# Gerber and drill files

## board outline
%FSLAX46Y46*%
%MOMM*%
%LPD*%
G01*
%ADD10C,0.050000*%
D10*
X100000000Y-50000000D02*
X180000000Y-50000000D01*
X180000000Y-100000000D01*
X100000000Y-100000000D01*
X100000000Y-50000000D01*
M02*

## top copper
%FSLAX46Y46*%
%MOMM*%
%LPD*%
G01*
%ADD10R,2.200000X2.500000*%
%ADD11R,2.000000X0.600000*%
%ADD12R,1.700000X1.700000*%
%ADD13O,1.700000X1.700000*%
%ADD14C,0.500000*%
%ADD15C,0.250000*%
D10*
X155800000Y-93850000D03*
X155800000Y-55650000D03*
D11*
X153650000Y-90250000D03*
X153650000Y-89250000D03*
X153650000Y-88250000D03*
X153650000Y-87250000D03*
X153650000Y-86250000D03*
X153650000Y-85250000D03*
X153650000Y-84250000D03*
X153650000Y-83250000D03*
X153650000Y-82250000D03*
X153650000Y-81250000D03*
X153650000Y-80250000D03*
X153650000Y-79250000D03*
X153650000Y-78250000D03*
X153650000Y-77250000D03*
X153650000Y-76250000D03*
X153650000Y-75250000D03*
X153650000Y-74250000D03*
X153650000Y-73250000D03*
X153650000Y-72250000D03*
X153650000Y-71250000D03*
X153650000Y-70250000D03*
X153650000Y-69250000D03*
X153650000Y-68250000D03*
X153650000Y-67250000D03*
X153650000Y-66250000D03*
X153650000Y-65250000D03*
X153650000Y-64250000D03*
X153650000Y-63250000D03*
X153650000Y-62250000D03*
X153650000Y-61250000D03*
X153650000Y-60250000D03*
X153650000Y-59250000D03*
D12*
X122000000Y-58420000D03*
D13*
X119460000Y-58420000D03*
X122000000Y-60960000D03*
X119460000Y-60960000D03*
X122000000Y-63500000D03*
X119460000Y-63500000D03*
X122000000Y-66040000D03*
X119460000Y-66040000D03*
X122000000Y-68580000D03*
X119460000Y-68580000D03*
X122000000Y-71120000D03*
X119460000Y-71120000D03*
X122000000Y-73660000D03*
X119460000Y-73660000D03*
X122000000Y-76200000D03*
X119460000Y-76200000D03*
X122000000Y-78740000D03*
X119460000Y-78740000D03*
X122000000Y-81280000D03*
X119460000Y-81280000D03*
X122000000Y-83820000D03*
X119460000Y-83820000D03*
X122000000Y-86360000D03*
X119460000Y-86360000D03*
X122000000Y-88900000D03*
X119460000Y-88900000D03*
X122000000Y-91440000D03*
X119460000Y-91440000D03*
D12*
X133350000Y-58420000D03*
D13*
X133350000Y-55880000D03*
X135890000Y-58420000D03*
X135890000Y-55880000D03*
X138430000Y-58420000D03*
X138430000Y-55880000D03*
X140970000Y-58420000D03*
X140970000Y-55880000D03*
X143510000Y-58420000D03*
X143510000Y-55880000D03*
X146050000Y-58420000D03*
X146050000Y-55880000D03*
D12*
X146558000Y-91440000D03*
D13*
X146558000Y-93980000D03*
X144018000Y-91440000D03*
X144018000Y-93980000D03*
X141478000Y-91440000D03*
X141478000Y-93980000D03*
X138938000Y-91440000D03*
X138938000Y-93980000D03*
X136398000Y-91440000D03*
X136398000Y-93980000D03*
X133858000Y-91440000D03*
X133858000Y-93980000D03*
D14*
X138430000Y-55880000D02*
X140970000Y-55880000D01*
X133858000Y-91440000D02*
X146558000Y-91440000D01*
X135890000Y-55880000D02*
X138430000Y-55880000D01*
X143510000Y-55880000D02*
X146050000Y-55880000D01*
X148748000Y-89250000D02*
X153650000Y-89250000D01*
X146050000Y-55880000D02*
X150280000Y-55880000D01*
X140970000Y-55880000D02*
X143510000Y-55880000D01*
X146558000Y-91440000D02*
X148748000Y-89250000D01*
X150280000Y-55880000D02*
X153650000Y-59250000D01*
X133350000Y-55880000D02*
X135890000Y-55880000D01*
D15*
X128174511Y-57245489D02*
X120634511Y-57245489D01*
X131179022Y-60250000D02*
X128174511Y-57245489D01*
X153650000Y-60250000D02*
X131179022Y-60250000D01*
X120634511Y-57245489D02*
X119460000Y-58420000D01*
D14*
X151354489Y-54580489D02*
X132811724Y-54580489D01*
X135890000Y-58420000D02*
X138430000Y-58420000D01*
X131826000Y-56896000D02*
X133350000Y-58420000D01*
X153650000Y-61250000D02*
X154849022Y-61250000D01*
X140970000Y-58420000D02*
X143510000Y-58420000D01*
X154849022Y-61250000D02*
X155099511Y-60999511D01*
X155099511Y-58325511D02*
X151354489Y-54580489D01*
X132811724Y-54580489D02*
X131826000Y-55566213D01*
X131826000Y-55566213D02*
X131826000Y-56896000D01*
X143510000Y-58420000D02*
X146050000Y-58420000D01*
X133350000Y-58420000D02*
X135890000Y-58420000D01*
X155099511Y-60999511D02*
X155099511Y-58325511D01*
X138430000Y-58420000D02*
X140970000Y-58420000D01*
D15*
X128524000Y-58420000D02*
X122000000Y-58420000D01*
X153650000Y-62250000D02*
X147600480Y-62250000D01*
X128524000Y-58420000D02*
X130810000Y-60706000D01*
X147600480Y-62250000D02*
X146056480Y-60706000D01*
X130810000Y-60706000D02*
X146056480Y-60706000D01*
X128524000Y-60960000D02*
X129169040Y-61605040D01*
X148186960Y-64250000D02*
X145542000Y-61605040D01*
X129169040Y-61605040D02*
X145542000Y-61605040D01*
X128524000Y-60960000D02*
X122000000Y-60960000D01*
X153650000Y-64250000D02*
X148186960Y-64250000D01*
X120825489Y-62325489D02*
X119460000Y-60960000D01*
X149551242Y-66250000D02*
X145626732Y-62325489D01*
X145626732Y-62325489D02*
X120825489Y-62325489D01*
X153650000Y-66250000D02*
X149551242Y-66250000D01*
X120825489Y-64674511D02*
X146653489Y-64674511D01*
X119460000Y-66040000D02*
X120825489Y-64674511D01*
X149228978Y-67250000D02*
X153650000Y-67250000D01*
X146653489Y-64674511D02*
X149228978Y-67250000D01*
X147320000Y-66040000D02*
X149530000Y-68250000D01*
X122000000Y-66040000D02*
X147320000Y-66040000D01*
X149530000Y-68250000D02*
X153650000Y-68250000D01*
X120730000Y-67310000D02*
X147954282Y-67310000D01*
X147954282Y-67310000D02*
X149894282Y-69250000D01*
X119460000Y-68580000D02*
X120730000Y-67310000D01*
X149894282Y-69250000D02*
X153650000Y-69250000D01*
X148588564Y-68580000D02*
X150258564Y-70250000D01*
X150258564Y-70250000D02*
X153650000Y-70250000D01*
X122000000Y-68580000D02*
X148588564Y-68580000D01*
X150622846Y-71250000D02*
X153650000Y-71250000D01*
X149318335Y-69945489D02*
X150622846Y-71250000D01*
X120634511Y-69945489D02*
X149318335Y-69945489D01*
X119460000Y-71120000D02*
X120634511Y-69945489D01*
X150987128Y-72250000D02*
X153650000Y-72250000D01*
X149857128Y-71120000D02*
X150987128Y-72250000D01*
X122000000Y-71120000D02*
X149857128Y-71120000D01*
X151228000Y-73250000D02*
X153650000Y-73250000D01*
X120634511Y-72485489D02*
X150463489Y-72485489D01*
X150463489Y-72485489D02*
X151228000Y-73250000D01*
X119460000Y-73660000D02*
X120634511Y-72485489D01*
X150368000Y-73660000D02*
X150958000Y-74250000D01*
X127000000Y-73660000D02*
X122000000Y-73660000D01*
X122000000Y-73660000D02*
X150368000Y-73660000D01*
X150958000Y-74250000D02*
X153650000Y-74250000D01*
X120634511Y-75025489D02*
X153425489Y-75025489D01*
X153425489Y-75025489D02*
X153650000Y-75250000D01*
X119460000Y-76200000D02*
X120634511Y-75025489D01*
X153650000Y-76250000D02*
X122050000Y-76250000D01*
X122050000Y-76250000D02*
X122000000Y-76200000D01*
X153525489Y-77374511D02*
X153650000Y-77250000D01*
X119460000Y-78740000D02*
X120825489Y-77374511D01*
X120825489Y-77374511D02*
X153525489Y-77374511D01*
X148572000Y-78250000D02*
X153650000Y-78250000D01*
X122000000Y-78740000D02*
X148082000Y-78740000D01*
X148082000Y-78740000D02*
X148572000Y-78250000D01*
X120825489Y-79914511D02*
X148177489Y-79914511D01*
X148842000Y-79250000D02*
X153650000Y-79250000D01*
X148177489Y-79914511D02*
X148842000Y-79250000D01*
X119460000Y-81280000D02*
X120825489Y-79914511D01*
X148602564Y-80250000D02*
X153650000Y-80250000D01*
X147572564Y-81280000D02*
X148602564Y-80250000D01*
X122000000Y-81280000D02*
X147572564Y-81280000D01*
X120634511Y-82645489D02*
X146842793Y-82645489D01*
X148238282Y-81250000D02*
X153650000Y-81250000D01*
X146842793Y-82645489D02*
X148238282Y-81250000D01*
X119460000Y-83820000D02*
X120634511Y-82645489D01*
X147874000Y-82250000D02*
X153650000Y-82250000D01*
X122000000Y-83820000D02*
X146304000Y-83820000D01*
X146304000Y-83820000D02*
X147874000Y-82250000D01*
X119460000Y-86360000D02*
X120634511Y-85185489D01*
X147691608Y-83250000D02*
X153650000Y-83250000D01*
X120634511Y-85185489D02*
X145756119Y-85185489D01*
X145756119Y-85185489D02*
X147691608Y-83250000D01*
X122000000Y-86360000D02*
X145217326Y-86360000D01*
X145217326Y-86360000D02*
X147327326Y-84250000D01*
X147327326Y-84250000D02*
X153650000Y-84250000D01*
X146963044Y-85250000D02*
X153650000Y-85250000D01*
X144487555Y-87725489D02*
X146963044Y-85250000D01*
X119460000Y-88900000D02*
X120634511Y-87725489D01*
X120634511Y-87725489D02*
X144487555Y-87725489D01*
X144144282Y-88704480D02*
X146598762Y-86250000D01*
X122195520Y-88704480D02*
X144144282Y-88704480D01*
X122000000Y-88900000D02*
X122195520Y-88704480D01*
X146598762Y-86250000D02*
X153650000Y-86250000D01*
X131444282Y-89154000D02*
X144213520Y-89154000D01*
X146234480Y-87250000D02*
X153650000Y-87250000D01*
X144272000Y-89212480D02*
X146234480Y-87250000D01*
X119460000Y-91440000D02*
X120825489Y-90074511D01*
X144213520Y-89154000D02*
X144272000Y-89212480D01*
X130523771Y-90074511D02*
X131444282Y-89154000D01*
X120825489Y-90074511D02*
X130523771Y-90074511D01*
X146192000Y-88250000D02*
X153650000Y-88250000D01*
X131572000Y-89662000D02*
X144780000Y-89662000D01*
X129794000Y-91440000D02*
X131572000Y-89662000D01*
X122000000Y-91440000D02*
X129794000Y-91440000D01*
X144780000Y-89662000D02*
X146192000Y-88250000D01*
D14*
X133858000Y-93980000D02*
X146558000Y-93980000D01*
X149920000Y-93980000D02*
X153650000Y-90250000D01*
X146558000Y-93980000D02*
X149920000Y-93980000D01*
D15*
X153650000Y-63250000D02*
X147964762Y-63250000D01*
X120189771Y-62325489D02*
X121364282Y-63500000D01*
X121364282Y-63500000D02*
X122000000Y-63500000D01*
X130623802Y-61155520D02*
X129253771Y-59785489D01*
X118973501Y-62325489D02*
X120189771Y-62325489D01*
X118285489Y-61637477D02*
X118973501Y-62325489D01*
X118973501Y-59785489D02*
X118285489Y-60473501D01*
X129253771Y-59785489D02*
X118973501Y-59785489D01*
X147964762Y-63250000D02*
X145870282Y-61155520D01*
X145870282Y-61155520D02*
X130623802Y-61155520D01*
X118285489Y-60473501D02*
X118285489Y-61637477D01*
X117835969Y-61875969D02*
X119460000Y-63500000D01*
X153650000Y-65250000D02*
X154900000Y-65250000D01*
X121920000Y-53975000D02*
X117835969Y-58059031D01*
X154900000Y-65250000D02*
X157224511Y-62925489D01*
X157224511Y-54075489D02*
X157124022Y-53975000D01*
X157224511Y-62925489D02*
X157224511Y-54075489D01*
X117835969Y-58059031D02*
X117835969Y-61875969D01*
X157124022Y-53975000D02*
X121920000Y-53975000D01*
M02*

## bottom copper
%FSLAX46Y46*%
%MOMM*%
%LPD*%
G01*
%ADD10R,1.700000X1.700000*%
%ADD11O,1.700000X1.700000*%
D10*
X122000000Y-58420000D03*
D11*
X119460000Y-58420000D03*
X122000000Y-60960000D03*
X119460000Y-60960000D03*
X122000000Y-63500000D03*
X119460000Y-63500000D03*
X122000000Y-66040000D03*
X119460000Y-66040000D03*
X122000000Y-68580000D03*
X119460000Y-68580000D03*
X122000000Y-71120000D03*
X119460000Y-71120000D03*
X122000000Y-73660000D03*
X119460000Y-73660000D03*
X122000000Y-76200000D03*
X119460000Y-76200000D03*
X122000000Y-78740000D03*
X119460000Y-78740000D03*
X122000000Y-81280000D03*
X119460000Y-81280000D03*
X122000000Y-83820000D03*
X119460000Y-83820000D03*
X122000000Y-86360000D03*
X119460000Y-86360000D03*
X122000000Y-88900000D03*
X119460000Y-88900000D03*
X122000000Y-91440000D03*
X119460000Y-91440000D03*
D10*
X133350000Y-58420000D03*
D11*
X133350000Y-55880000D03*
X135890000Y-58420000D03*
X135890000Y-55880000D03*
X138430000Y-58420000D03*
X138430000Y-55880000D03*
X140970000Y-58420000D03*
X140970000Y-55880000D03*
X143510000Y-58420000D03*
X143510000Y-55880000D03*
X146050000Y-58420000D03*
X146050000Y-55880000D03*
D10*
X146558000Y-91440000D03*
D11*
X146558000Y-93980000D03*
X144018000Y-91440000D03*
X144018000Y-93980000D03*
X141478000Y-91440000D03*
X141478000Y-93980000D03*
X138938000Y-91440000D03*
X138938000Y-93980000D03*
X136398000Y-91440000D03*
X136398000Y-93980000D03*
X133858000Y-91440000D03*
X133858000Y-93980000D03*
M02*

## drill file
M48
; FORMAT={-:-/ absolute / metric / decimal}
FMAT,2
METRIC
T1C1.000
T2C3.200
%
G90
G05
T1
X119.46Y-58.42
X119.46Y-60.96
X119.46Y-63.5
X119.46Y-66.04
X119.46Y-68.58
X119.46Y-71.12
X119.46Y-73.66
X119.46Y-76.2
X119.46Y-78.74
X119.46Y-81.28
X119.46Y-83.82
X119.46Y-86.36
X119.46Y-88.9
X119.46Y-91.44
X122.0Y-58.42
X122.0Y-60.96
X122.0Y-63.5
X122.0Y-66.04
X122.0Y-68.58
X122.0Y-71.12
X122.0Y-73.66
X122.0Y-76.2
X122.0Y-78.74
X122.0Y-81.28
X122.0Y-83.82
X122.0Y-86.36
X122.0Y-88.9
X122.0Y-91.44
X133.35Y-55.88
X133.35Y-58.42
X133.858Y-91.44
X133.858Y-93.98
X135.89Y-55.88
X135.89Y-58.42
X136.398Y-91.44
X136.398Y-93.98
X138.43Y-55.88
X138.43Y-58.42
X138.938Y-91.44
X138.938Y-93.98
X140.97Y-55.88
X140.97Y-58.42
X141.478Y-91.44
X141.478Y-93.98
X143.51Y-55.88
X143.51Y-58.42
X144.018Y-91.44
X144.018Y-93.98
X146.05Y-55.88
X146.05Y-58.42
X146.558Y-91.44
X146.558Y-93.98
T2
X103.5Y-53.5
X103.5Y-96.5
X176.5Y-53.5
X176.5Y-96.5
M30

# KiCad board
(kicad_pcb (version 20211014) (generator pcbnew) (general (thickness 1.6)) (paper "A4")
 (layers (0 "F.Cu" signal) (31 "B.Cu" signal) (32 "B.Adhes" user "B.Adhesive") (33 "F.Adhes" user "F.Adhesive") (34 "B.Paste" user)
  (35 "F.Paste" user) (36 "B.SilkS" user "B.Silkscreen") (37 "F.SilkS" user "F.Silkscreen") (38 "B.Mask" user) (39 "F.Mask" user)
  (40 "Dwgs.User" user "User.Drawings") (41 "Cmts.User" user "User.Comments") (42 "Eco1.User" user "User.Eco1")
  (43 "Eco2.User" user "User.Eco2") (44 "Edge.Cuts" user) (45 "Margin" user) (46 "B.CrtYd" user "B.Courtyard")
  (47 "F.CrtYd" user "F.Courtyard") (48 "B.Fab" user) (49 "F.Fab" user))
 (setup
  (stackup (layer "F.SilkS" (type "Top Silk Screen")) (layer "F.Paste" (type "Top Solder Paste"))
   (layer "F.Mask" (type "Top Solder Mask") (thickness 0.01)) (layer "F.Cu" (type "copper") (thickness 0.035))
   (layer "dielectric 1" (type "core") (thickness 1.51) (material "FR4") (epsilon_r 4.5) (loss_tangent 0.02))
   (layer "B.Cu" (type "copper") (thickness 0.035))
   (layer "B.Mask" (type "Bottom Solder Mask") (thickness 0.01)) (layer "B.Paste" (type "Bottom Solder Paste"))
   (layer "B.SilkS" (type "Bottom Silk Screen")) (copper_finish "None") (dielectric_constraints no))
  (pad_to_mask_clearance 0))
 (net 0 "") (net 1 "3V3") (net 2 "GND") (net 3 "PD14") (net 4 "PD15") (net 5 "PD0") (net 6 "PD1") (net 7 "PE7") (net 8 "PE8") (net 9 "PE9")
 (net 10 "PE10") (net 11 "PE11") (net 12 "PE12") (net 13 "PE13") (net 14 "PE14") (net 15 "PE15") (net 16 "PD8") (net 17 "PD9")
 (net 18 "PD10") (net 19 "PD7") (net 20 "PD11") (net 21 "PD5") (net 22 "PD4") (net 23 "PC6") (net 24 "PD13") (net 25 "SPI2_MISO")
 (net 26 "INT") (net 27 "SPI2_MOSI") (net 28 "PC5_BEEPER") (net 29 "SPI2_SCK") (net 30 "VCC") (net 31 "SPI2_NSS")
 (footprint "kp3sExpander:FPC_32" (layer "F.Cu") (at 153.65 74.75 90)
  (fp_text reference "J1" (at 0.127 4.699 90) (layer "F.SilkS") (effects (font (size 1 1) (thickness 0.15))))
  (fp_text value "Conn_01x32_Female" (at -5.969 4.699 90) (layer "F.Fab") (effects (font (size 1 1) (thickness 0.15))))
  (pad "0" smd rect locked (at -19.1 2.15 90) (size 2.5 2.2) (layers "F.Cu" "F.Paste" "F.Mask"))
  (pad "0" smd rect locked (at 19.1 2.15 90) (size 2.5 2.2) (layers "F.Cu" "F.Paste" "F.Mask"))
  (pad "1" smd rect locked (at -15.5 0 90) (size 0.6 2) (layers "F.Cu" "F.Paste" "F.Mask") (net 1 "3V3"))
  (pad "2" smd rect locked (at -14.5 0 90) (size 0.6 2) (layers "F.Cu" "F.Paste" "F.Mask") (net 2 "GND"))
  (pad "3" smd rect locked (at -13.5 0 90) (size 0.6 2) (layers "F.Cu" "F.Paste" "F.Mask") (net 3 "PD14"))
  (pad "4" smd rect locked (at -12.5 0 90) (size 0.6 2) (layers "F.Cu" "F.Paste" "F.Mask") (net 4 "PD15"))
  (pad "5" smd rect locked (at -11.5 0 90) (size 0.6 2) (layers "F.Cu" "F.Paste" "F.Mask") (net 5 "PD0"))
  (pad "6" smd rect locked (at -10.5 0 90) (size 0.6 2) (layers "F.Cu" "F.Paste" "F.Mask") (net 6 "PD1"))
  (pad "7" smd rect locked (at -9.5 0 90) (size 0.6 2) (layers "F.Cu" "F.Paste" "F.Mask") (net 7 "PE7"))
  (pad "8" smd rect locked (at -8.5 0 90) (size 0.6 2) (layers "F.Cu" "F.Paste" "F.Mask") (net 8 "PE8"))
  (pad "9" smd rect locked (at -7.5 0 90) (size 0.6 2) (layers "F.Cu" "F.Paste" "F.Mask") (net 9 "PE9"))
  (pad "10" smd rect locked (at -6.5 0 90) (size 0.6 2) (layers "F.Cu" "F.Paste" "F.Mask") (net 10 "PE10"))
  (pad "11" smd rect locked (at -5.5 0 90) (size 0.6 2) (layers "F.Cu" "F.Paste" "F.Mask") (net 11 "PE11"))
  (pad "12" smd rect locked (at -4.5 0 90) (size 0.6 2) (layers "F.Cu" "F.Paste" "F.Mask") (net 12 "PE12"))
  (pad "13" smd rect locked (at -3.5 0 90) (size 0.6 2) (layers "F.Cu" "F.Paste" "F.Mask") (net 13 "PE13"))
  (pad "14" smd rect locked (at -2.5 0 90) (size 0.6 2) (layers "F.Cu" "F.Paste" "F.Mask") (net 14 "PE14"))
  (pad "15" smd rect locked (at -1.5 0 90) (size 0.6 2) (layers "F.Cu" "F.Paste" "F.Mask") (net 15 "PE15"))
  (pad "16" smd rect locked (at -0.5 0 90) (size 0.6 2) (layers "F.Cu" "F.Paste" "F.Mask") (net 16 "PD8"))
  (pad "17" smd rect locked (at 0.5 0 90) (size 0.6 2) (layers "F.Cu" "F.Paste" "F.Mask") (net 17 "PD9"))
  (pad "18" smd rect locked (at 1.5 0 90) (size 0.6 2) (layers "F.Cu" "F.Paste" "F.Mask") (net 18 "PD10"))
  (pad "19" smd rect locked (at 2.5 0 90) (size 0.6 2) (layers "F.Cu" "F.Paste" "F.Mask") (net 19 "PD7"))
  (pad "20" smd rect locked (at 3.5 0 90) (size 0.6 2) (layers "F.Cu" "F.Paste" "F.Mask") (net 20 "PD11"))
  (pad "21" smd rect locked (at 4.5 0 90) (size 0.6 2) (layers "F.Cu" "F.Paste" "F.Mask") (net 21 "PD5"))
  (pad "22" smd rect locked (at 5.5 0 90) (size 0.6 2) (layers "F.Cu" "F.Paste" "F.Mask") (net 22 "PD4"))
  (pad "23" smd rect locked (at 6.5 0 90) (size 0.6 2) (layers "F.Cu" "F.Paste" "F.Mask") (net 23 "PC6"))
  (pad "24" smd rect locked (at 7.5 0 90) (size 0.6 2) (layers "F.Cu" "F.Paste" "F.Mask") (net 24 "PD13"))
  (pad "25" smd rect locked (at 8.5 0 90) (size 0.6 2) (layers "F.Cu" "F.Paste" "F.Mask") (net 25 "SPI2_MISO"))
  (pad "26" smd rect locked (at 9.5 0 90) (size 0.6 2) (layers "F.Cu" "F.Paste" "F.Mask") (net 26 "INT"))
  (pad "27" smd rect locked (at 10.5 0 90) (size 0.6 2) (layers "F.Cu" "F.Paste" "F.Mask") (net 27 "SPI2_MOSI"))
  (pad "28" smd rect locked (at 11.5 0 90) (size 0.6 2) (layers "F.Cu" "F.Paste" "F.Mask") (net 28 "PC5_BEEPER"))
  (pad "29" smd rect locked (at 12.5 0 90) (size 0.6 2) (layers "F.Cu" "F.Paste" "F.Mask") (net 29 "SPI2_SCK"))
  (pad "30" smd rect locked (at 13.5 0 90) (size 0.6 2) (layers "F.Cu" "F.Paste" "F.Mask") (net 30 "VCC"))
  (pad "31" smd rect locked (at 14.5 0 90) (size 0.6 2) (layers "F.Cu" "F.Paste" "F.Mask") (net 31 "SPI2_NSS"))
  (pad "32" smd rect locked (at 15.5 0 90) (size 0.6 2) (layers "F.Cu" "F.Paste" "F.Mask") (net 2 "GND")))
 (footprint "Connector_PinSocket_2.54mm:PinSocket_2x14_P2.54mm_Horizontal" (layer "F.Cu") (at 122 58.42)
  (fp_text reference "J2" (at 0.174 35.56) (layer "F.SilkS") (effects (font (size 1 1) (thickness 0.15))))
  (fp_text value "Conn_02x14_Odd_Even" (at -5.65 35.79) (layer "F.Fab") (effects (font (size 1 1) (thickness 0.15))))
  (pad "1" thru_hole rect (at 0 0) (size 1.7 1.7) (drill 1) (layers *.Cu *.Mask) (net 29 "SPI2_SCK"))
  (pad "2" thru_hole oval (at -2.54 0) (size 1.7 1.7) (drill 1) (layers *.Cu *.Mask) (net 31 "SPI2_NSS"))
  (pad "3" thru_hole oval (at 0 2.54) (size 1.7 1.7) (drill 1) (layers *.Cu *.Mask) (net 27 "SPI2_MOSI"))
  (pad "4" thru_hole oval (at -2.54 2.54) (size 1.7 1.7) (drill 1) (layers *.Cu *.Mask) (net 25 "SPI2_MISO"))
  (pad "5" thru_hole oval (at 0 5.08) (size 1.7 1.7) (drill 1) (layers *.Cu *.Mask) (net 28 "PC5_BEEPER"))
  (pad "6" thru_hole oval (at -2.54 5.08) (size 1.7 1.7) (drill 1) (layers *.Cu *.Mask) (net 26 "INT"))
  (pad "7" thru_hole oval (at 0 7.62) (size 1.7 1.7) (drill 1) (layers *.Cu *.Mask) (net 23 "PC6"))
  (pad "8" thru_hole oval (at -2.54 7.62) (size 1.7 1.7) (drill 1) (layers *.Cu *.Mask) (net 24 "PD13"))
  (pad "9" thru_hole oval (at 0 10.16) (size 1.7 1.7) (drill 1) (layers *.Cu *.Mask) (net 21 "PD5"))
  (pad "10" thru_hole oval (at -2.54 10.16) (size 1.7 1.7) (drill 1) (layers *.Cu *.Mask) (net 22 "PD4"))
  (pad "11" thru_hole oval (at 0 12.7) (size 1.7 1.7) (drill 1) (layers *.Cu *.Mask) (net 19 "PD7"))
  (pad "12" thru_hole oval (at -2.54 12.7) (size 1.7 1.7) (drill 1) (layers *.Cu *.Mask) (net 20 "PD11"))
  (pad "13" thru_hole oval (at 0 15.24) (size 1.7 1.7) (drill 1) (layers *.Cu *.Mask) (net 17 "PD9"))
  (pad "14" thru_hole oval (at -2.54 15.24) (size 1.7 1.7) (drill 1) (layers *.Cu *.Mask) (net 18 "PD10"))
  (pad "15" thru_hole oval (at 0 17.78) (size 1.7 1.7) (drill 1) (layers *.Cu *.Mask) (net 15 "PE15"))
  (pad "16" thru_hole oval (at -2.54 17.78) (size 1.7 1.7) (drill 1) (layers *.Cu *.Mask) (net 16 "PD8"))
  (pad "17" thru_hole oval (at 0 20.32) (size 1.7 1.7) (drill 1) (layers *.Cu *.Mask) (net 13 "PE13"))
  (pad "18" thru_hole oval (at -2.54 20.32) (size 1.7 1.7) (drill 1) (layers *.Cu *.Mask) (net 14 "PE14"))
  (pad "19" thru_hole oval (at 0 22.86) (size 1.7 1.7) (drill 1) (layers *.Cu *.Mask) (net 11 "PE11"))
  (pad "20" thru_hole oval (at -2.54 22.86) (size 1.7 1.7) (drill 1) (layers *.Cu *.Mask) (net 12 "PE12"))
  (pad "21" thru_hole oval (at 0 25.4) (size 1.7 1.7) (drill 1) (layers *.Cu *.Mask) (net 9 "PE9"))
  (pad "22" thru_hole oval (at -2.54 25.4) (size 1.7 1.7) (drill 1) (layers *.Cu *.Mask) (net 10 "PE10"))
  (pad "23" thru_hole oval (at 0 27.94) (size 1.7 1.7) (drill 1) (layers *.Cu *.Mask) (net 7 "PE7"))
  (pad "24" thru_hole oval (at -2.54 27.94) (size 1.7 1.7) (drill 1) (layers *.Cu *.Mask) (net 8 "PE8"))
  (pad "25" thru_hole oval (at 0 30.48) (size 1.7 1.7) (drill 1) (layers *.Cu *.Mask) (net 5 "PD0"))
  (pad "26" thru_hole oval (at -2.54 30.48) (size 1.7 1.7) (drill 1) (layers *.Cu *.Mask) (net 6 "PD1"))
  (pad "27" thru_hole oval (at 0 33.02) (size 1.7 1.7) (drill 1) (layers *.Cu *.Mask) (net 3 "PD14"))
  (pad "28" thru_hole oval (at -2.54 33.02) (size 1.7 1.7) (drill 1) (layers *.Cu *.Mask) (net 4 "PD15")))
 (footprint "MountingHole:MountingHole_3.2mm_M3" (layer "F.Cu") (at 103.5 96.5)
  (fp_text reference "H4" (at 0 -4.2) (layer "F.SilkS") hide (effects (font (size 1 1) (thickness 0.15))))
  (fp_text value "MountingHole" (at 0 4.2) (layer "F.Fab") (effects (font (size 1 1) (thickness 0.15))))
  (pad "" np_thru_hole circle locked (at 0 0) (size 3.2 3.2) (drill 3.2) (layers *.Cu *.Mask)))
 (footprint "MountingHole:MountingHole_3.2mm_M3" (layer "F.Cu") (at 103.5 53.5)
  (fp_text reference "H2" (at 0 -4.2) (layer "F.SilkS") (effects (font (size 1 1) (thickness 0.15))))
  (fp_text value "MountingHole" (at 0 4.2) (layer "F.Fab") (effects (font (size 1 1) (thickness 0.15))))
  (pad "" np_thru_hole circle locked (at 0 0) (size 3.2 3.2) (drill 3.2) (layers *.Cu *.Mask)))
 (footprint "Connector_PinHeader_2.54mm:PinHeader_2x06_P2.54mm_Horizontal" (layer "F.Cu") (at 133.35 58.42 90)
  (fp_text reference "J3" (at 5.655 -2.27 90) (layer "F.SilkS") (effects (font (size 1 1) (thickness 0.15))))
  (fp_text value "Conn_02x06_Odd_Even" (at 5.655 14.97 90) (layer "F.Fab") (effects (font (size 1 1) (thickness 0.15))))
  (pad "1" thru_hole rect (at 0 0 90) (size 1.7 1.7) (drill 1) (layers *.Cu *.Mask) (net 30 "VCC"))
  (pad "2" thru_hole oval (at 2.54 0 90) (size 1.7 1.7) (drill 1) (layers *.Cu *.Mask) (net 2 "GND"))
  (pad "3" thru_hole oval (at 0 2.54 90) (size 1.7 1.7) (drill 1) (layers *.Cu *.Mask) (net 30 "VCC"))
  (pad "4" thru_hole oval (at 2.54 2.54 90) (size 1.7 1.7) (drill 1) (layers *.Cu *.Mask) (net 2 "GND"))
  (pad "5" thru_hole oval (at 0 5.08 90) (size 1.7 1.7) (drill 1) (layers *.Cu *.Mask) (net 30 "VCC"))
  (pad "6" thru_hole oval (at 2.54 5.08 90) (size 1.7 1.7) (drill 1) (layers *.Cu *.Mask) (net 2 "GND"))
  (pad "7" thru_hole oval (at 0 7.62 90) (size 1.7 1.7) (drill 1) (layers *.Cu *.Mask) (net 30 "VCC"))
  (pad "8" thru_hole oval (at 2.54 7.62 90) (size 1.7 1.7) (drill 1) (layers *.Cu *.Mask) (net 2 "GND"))
  (pad "9" thru_hole oval (at 0 10.16 90) (size 1.7 1.7) (drill 1) (layers *.Cu *.Mask) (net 30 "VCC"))
  (pad "10" thru_hole oval (at 2.54 10.16 90) (size 1.7 1.7) (drill 1) (layers *.Cu *.Mask) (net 2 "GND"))
  (pad "11" thru_hole oval (at 0 12.7 90) (size 1.7 1.7) (drill 1) (layers *.Cu *.Mask) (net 30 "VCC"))
  (pad "12" thru_hole oval (at 2.54 12.7 90) (size 1.7 1.7) (drill 1) (layers *.Cu *.Mask) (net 2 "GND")))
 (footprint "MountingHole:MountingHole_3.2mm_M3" (layer "F.Cu") (at 176.5 96.5)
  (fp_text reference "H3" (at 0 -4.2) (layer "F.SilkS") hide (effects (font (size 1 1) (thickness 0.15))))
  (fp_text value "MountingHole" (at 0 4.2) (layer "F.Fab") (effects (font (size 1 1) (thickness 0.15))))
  (pad "" np_thru_hole circle locked (at 0 0) (size 3.2 3.2) (drill 3.2) (layers *.Cu *.Mask)))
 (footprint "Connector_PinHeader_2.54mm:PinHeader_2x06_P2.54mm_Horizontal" (layer "F.Cu") (at 146.558 91.44 -90)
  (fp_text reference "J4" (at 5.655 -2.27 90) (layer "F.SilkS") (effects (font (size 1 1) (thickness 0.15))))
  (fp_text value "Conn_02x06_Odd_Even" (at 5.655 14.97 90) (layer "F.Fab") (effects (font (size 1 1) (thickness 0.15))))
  (pad "1" thru_hole rect (at 0 0 270) (size 1.7 1.7) (drill 1) (layers *.Cu *.Mask) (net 2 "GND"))
  (pad "2" thru_hole oval (at 2.54 0 270) (size 1.7 1.7) (drill 1) (layers *.Cu *.Mask) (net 1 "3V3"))
  (pad "3" thru_hole oval (at 0 2.54 270) (size 1.7 1.7) (drill 1) (layers *.Cu *.Mask) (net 2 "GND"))
  (pad "4" thru_hole oval (at 2.54 2.54 270) (size 1.7 1.7) (drill 1) (layers *.Cu *.Mask) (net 1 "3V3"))
  (pad "5" thru_hole oval (at 0 5.08 270) (size 1.7 1.7) (drill 1) (layers *.Cu *.Mask) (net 2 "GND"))
  (pad "6" thru_hole oval (at 2.54 5.08 270) (size 1.7 1.7) (drill 1) (layers *.Cu *.Mask) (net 1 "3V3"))
  (pad "7" thru_hole oval (at 0 7.62 270) (size 1.7 1.7) (drill 1) (layers *.Cu *.Mask) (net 2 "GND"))
  (pad "8" thru_hole oval (at 2.54 7.62 270) (size 1.7 1.7) (drill 1) (layers *.Cu *.Mask) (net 1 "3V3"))
  (pad "9" thru_hole oval (at 0 10.16 270) (size 1.7 1.7) (drill 1) (layers *.Cu *.Mask) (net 2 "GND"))
  (pad "10" thru_hole oval (at 2.54 10.16 270) (size 1.7 1.7) (drill 1) (layers *.Cu *.Mask) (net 1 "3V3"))
  (pad "11" thru_hole oval (at 0 12.7 270) (size 1.7 1.7) (drill 1) (layers *.Cu *.Mask) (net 2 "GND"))
  (pad "12" thru_hole oval (at 2.54 12.7 270) (size 1.7 1.7) (drill 1) (layers *.Cu *.Mask) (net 1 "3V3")))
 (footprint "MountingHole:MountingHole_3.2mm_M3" (layer "F.Cu") (at 176.5 53.5)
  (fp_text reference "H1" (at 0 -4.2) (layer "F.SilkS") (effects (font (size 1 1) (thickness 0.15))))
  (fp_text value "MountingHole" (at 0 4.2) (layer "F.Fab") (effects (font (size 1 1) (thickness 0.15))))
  (pad "" np_thru_hole circle locked (at 0 0) (size 3.2 3.2) (drill 3.2) (layers *.Cu *.Mask)))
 (gr_rect (start 100 50) (end 180 100) (layer "Edge.Cuts") (width 0.05) (fill none))
 (segment (start 138.43 55.88) (end 140.97 55.88) (width 0.5) (layer "F.Cu") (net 2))
 (segment (start 133.858 91.44) (end 146.558 91.44) (width 0.5) (layer "F.Cu") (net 2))
 (segment (start 135.89 55.88) (end 138.43 55.88) (width 0.5) (layer "F.Cu") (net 2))
 (segment (start 143.51 55.88) (end 146.05 55.88) (width 0.5) (layer "F.Cu") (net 2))
 (segment (start 148.748 89.25) (end 153.65 89.25) (width 0.5) (layer "F.Cu") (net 2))
 (segment (start 146.05 55.88) (end 150.28 55.88) (width 0.5) (layer "F.Cu") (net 2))
 (segment (start 140.97 55.88) (end 143.51 55.88) (width 0.5) (layer "F.Cu") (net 2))
 (segment (start 146.558 91.44) (end 148.748 89.25) (width 0.5) (layer "F.Cu") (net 2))
 (segment (start 150.28 55.88) (end 153.65 59.25) (width 0.5) (layer "F.Cu") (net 2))
 (segment (start 133.35 55.88) (end 135.89 55.88) (width 0.5) (layer "F.Cu") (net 2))
 (segment (start 128.174511 57.245489) (end 120.634511 57.245489) (width 0.25) (layer "F.Cu") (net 31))
 (segment (start 131.179022 60.25) (end 128.174511 57.245489) (width 0.25) (layer "F.Cu") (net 31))
 (segment (start 153.65 60.25) (end 131.179022 60.25) (width 0.25) (layer "F.Cu") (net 31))
 (segment (start 120.634511 57.245489) (end 119.46 58.42) (width 0.25) (layer "F.Cu") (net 31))
 (segment (start 151.354489 54.580489) (end 132.811724 54.580489) (width 0.5) (layer "F.Cu") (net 30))
 (segment (start 135.89 58.42) (end 138.43 58.42) (width 0.5) (layer "F.Cu") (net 30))
 (segment (start 131.826 56.896) (end 133.35 58.42) (width 0.5) (layer "F.Cu") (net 30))
 (segment (start 153.65 61.25) (end 154.849022 61.25) (width 0.5) (layer "F.Cu") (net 30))
 (segment (start 140.97 58.42) (end 143.51 58.42) (width 0.5) (layer "F.Cu") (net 30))
 (segment (start 154.849022 61.25) (end 155.099511 60.999511) (width 0.5) (layer "F.Cu") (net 30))
 (segment (start 155.099511 58.325511) (end 151.354489 54.580489) (width 0.5) (layer "F.Cu") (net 30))
 (segment (start 132.811724 54.580489) (end 131.826 55.566213) (width 0.5) (layer "F.Cu") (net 30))
 (segment (start 131.826 55.566213) (end 131.826 56.896) (width 0.5) (layer "F.Cu") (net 30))
 (segment (start 143.51 58.42) (end 146.05 58.42) (width 0.5) (layer "F.Cu") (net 30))
 (segment (start 133.35 58.42) (end 135.89 58.42) (width 0.5) (layer "F.Cu") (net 30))
 (segment (start 155.099511 60.999511) (end 155.099511 58.325511) (width 0.5) (layer "F.Cu") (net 30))
 (segment (start 138.43 58.42) (end 140.97 58.42) (width 0.5) (layer "F.Cu") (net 30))
 (segment (start 128.524 58.42) (end 122 58.42) (width 0.25) (layer "F.Cu") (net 29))
 (segment (start 153.65 62.25) (end 147.60048 62.25) (width 0.25) (layer "F.Cu") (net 29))
 (segment (start 128.524 58.42) (end 130.81 60.706) (width 0.25) (layer "F.Cu") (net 29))
 (segment (start 147.60048 62.25) (end 146.05648 60.706) (width 0.25) (layer "F.Cu") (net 29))
 (segment (start 130.81 60.706) (end 146.05648 60.706) (width 0.25) (layer "F.Cu") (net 29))
 (segment (start 128.524 60.96) (end 129.16904 61.60504) (width 0.25) (layer "F.Cu") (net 27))
 (segment (start 148.18696 64.25) (end 145.542 61.60504) (width 0.25) (layer "F.Cu") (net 27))
 (segment (start 129.16904 61.60504) (end 145.542 61.60504) (width 0.25) (layer "F.Cu") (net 27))
 (segment (start 128.524 60.96) (end 122 60.96) (width 0.25) (layer "F.Cu") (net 27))
 (segment (start 153.65 64.25) (end 148.18696 64.25) (width 0.25) (layer "F.Cu") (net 27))
 (segment (start 120.825489 62.325489) (end 119.46 60.96) (width 0.25) (layer "F.Cu") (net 25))
 (segment (start 149.551242 66.25) (end 145.626732 62.325489) (width 0.25) (layer "F.Cu") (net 25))
 (segment (start 145.626732 62.325489) (end 120.825489 62.325489) (width 0.25) (layer "F.Cu") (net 25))
 (segment (start 153.65 66.25) (end 149.551242 66.25) (width 0.25) (layer "F.Cu") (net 25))
 (segment (start 120.825489 64.674511) (end 146.653489 64.674511) (width 0.25) (layer "F.Cu") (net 24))
 (segment (start 119.46 66.04) (end 120.825489 64.674511) (width 0.25) (layer "F.Cu") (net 24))
 (segment (start 149.228978 67.25) (end 153.65 67.25) (width 0.25) (layer "F.Cu") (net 24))
 (segment (start 146.653489 64.674511) (end 149.228978 67.25) (width 0.25) (layer "F.Cu") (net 24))
 (segment (start 147.32 66.04) (end 149.53 68.25) (width 0.25) (layer "F.Cu") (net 23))
 (segment (start 122 66.04) (end 147.32 66.04) (width 0.25) (layer "F.Cu") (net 23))
 (segment (start 149.53 68.25) (end 153.65 68.25) (width 0.25) (layer "F.Cu") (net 23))
 (segment (start 120.73 67.31) (end 147.954282 67.31) (width 0.25) (layer "F.Cu") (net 22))
 (segment (start 147.954282 67.31) (end 149.894282 69.25) (width 0.25) (layer "F.Cu") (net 22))
 (segment (start 119.46 68.58) (end 120.73 67.31) (width 0.25) (layer "F.Cu") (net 22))
 (segment (start 149.894282 69.25) (end 153.65 69.25) (width 0.25) (layer "F.Cu") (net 22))
 (segment (start 148.588564 68.58) (end 150.258564 70.25) (width 0.25) (layer "F.Cu") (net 21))
 (segment (start 150.258564 70.25) (end 153.65 70.25) (width 0.25) (layer "F.Cu") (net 21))
 (segment (start 122 68.58) (end 148.588564 68.58) (width 0.25) (layer "F.Cu") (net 21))
 (segment (start 150.622846 71.25) (end 153.65 71.25) (width 0.25) (layer "F.Cu") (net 20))
 (segment (start 149.318335 69.945489) (end 150.622846 71.25) (width 0.25) (layer "F.Cu") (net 20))
 (segment (start 120.634511 69.945489) (end 149.318335 69.945489) (width 0.25) (layer "F.Cu") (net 20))
 (segment (start 119.46 71.12) (end 120.634511 69.945489) (width 0.25) (layer "F.Cu") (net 20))
 (segment (start 150.987128 72.25) (end 153.65 72.25) (width 0.25) (layer "F.Cu") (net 19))
 (segment (start 149.857128 71.12) (end 150.987128 72.25) (width 0.25) (layer "F.Cu") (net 19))
 (segment (start 122 71.12) (end 149.857128 71.12) (width 0.25) (layer "F.Cu") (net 19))
 (segment (start 151.228 73.25) (end 153.65 73.25) (width 0.25) (layer "F.Cu") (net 18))
 (segment (start 120.634511 72.485489) (end 150.463489 72.485489) (width 0.25) (layer "F.Cu") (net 18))
 (segment (start 150.463489 72.485489) (end 151.228 73.25) (width 0.25) (layer "F.Cu") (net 18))
 (segment (start 119.46 73.66) (end 120.634511 72.485489) (width 0.25) (layer "F.Cu") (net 18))
 (segment (start 150.368 73.66) (end 150.958 74.25) (width 0.25) (layer "F.Cu") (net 17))
 (segment (start 127 73.66) (end 122 73.66) (width 0.25) (layer "F.Cu") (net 17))
 (segment (start 122 73.66) (end 150.368 73.66) (width 0.25) (layer "F.Cu") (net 17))
 (segment (start 150.958 74.25) (end 153.65 74.25) (width 0.25) (layer "F.Cu") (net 17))
 (segment (start 120.634511 75.025489) (end 153.425489 75.025489) (width 0.25) (layer "F.Cu") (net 16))
 (segment (start 153.425489 75.025489) (end 153.65 75.25) (width 0.25) (layer "F.Cu") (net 16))
 (segment (start 119.46 76.2) (end 120.634511 75.025489) (width 0.25) (layer "F.Cu") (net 16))
 (segment (start 153.65 76.25) (end 122.05 76.25) (width 0.25) (layer "F.Cu") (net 15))
 (segment (start 122.05 76.25) (end 122 76.2) (width 0.25) (layer "F.Cu") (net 15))
 (segment (start 153.525489 77.374511) (end 153.65 77.25) (width 0.25) (layer "F.Cu") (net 14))
 (segment (start 119.46 78.74) (end 120.825489 77.374511) (width 0.25) (layer "F.Cu") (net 14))
 (segment (start 120.825489 77.374511) (end 153.525489 77.374511) (width 0.25) (layer "F.Cu") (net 14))
 (segment (start 148.572 78.25) (end 153.65 78.25) (width 0.25) (layer "F.Cu") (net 13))
 (segment (start 122 78.74) (end 148.082 78.74) (width 0.25) (layer "F.Cu") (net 13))
 (segment (start 148.082 78.74) (end 148.572 78.25) (width 0.25) (layer "F.Cu") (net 13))
 (segment (start 120.825489 79.914511) (end 148.177489 79.914511) (width 0.25) (layer "F.Cu") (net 12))
 (segment (start 148.842 79.25) (end 153.65 79.25) (width 0.25) (layer "F.Cu") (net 12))
 (segment (start 148.177489 79.914511) (end 148.842 79.25) (width 0.25) (layer "F.Cu") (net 12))
 (segment (start 119.46 81.28) (end 120.825489 79.914511) (width 0.25) (layer "F.Cu") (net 12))
 (segment (start 148.602564 80.25) (end 153.65 80.25) (width 0.25) (layer "F.Cu") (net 11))
 (segment (start 147.572564 81.28) (end 148.602564 80.25) (width 0.25) (layer "F.Cu") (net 11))
 (segment (start 122 81.28) (end 147.572564 81.28) (width 0.25) (layer "F.Cu") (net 11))
 (segment (start 120.634511 82.645489) (end 146.842793 82.645489) (width 0.25) (layer "F.Cu") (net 10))
 (segment (start 148.238282 81.25) (end 153.65 81.25) (width 0.25) (layer "F.Cu") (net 10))
 (segment (start 146.842793 82.645489) (end 148.238282 81.25) (width 0.25) (layer "F.Cu") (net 10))
 (segment (start 119.46 83.82) (end 120.634511 82.645489) (width 0.25) (layer "F.Cu") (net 10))
 (segment (start 147.874 82.25) (end 153.65 82.25) (width 0.25) (layer "F.Cu") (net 9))
 (segment (start 122 83.82) (end 146.304 83.82) (width 0.25) (layer "F.Cu") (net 9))
 (segment (start 146.304 83.82) (end 147.874 82.25) (width 0.25) (layer "F.Cu") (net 9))
 (segment (start 119.46 86.36) (end 120.634511 85.185489) (width 0.25) (layer "F.Cu") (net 8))
 (segment (start 147.691608 83.25) (end 153.65 83.25) (width 0.25) (layer "F.Cu") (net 8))
 (segment (start 120.634511 85.185489) (end 145.756119 85.185489) (width 0.25) (layer "F.Cu") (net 8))
 (segment (start 145.756119 85.185489) (end 147.691608 83.25) (width 0.25) (layer "F.Cu") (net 8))
 (segment (start 122 86.36) (end 145.217326 86.36) (width 0.25) (layer "F.Cu") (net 7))
 (segment (start 145.217326 86.36) (end 147.327326 84.25) (width 0.25) (layer "F.Cu") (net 7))
 (segment (start 147.327326 84.25) (end 153.65 84.25) (width 0.25) (layer "F.Cu") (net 7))
 (segment (start 146.963044 85.25) (end 153.65 85.25) (width 0.25) (layer "F.Cu") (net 6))
 (segment (start 144.487555 87.725489) (end 146.963044 85.25) (width 0.25) (layer "F.Cu") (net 6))
 (segment (start 119.46 88.9) (end 120.634511 87.725489) (width 0.25) (layer "F.Cu") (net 6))
 (segment (start 120.634511 87.725489) (end 144.487555 87.725489) (width 0.25) (layer "F.Cu") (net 6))
 (segment (start 144.144282 88.70448) (end 146.598762 86.25) (width 0.25) (layer "F.Cu") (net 5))
 (segment (start 122.19552 88.70448) (end 144.144282 88.70448) (width 0.25) (layer "F.Cu") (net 5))
 (segment (start 122 88.9) (end 122.19552 88.70448) (width 0.25) (layer "F.Cu") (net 5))
 (segment (start 146.598762 86.25) (end 153.65 86.25) (width 0.25) (layer "F.Cu") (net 5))
 (segment (start 131.444282 89.154) (end 144.21352 89.154) (width 0.25) (layer "F.Cu") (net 4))
 (segment (start 146.23448 87.25) (end 153.65 87.25) (width 0.25) (layer "F.Cu") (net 4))
 (segment (start 144.272 89.21248) (end 146.23448 87.25) (width 0.25) (layer "F.Cu") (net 4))
 (segment (start 119.46 91.44) (end 120.825489 90.074511) (width 0.25) (layer "F.Cu") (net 4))
 (segment (start 144.21352 89.154) (end 144.272 89.21248) (width 0.25) (layer "F.Cu") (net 4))
 (segment (start 130.523771 90.074511) (end 131.444282 89.154) (width 0.25) (layer "F.Cu") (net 4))
 (segment (start 120.825489 90.074511) (end 130.523771 90.074511) (width 0.25) (layer "F.Cu") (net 4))
 (segment (start 146.192 88.25) (end 153.65 88.25) (width 0.25) (layer "F.Cu") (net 3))
 (segment (start 131.572 89.662) (end 144.78 89.662) (width 0.25) (layer "F.Cu") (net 3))
 (segment (start 129.794 91.44) (end 131.572 89.662) (width 0.25) (layer "F.Cu") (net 3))
 (segment (start 122 91.44) (end 129.794 91.44) (width 0.25) (layer "F.Cu") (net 3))
 (segment (start 144.78 89.662) (end 146.192 88.25) (width 0.25) (layer "F.Cu") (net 3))
 (segment (start 133.858 93.98) (end 146.558 93.98) (width 0.5) (layer "F.Cu") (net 1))
 (segment (start 149.92 93.98) (end 153.65 90.25) (width 0.5) (layer "F.Cu") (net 1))
 (segment (start 146.558 93.98) (end 149.92 93.98) (width 0.5) (layer "F.Cu") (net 1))
 (segment (start 153.65 63.25) (end 147.964762 63.25) (width 0.25) (layer "F.Cu") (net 28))
 (segment (start 120.189771 62.325489) (end 121.364282 63.5) (width 0.25) (layer "F.Cu") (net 28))
 (segment (start 121.364282 63.5) (end 122 63.5) (width 0.25) (layer "F.Cu") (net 28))
 (segment (start 130.623802 61.15552) (end 129.253771 59.785489) (width 0.25) (layer "F.Cu") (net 28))
 (segment (start 118.973501 62.325489) (end 120.189771 62.325489) (width 0.25) (layer "F.Cu") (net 28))
 (segment (start 118.285489 61.637477) (end 118.973501 62.325489) (width 0.25) (layer "F.Cu") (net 28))
 (segment (start 118.973501 59.785489) (end 118.285489 60.473501) (width 0.25) (layer "F.Cu") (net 28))
 (segment (start 129.253771 59.785489) (end 118.973501 59.785489) (width 0.25) (layer "F.Cu") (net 28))
 (segment (start 147.964762 63.25) (end 145.870282 61.15552) (width 0.25) (layer "F.Cu") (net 28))
 (segment (start 145.870282 61.15552) (end 130.623802 61.15552) (width 0.25) (layer "F.Cu") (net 28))
 (segment (start 118.285489 60.473501) (end 118.285489 61.637477) (width 0.25) (layer "F.Cu") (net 28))
 (segment (start 117.835969 61.875969) (end 119.46 63.5) (width 0.25) (layer "F.Cu") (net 26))
 (segment (start 153.65 65.25) (end 154.9 65.25) (width 0.25) (layer "F.Cu") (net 26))
 (segment (start 121.92 53.975) (end 117.835969 58.059031) (width 0.25) (layer "F.Cu") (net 26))
 (segment (start 154.9 65.25) (end 157.224511 62.925489) (width 0.25) (layer "F.Cu") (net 26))
 (segment (start 157.224511 54.075489) (end 157.124022 53.975) (width 0.25) (layer "F.Cu") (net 26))
 (segment (start 157.224511 62.925489) (end 157.224511 54.075489) (width 0.25) (layer "F.Cu") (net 26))
 (segment (start 117.835969 58.059031) (end 117.835969 61.875969) (width 0.25) (layer "F.Cu") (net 26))
 (segment (start 157.124022 53.975) (end 121.92 53.975) (width 0.25) (layer "F.Cu") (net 26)))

